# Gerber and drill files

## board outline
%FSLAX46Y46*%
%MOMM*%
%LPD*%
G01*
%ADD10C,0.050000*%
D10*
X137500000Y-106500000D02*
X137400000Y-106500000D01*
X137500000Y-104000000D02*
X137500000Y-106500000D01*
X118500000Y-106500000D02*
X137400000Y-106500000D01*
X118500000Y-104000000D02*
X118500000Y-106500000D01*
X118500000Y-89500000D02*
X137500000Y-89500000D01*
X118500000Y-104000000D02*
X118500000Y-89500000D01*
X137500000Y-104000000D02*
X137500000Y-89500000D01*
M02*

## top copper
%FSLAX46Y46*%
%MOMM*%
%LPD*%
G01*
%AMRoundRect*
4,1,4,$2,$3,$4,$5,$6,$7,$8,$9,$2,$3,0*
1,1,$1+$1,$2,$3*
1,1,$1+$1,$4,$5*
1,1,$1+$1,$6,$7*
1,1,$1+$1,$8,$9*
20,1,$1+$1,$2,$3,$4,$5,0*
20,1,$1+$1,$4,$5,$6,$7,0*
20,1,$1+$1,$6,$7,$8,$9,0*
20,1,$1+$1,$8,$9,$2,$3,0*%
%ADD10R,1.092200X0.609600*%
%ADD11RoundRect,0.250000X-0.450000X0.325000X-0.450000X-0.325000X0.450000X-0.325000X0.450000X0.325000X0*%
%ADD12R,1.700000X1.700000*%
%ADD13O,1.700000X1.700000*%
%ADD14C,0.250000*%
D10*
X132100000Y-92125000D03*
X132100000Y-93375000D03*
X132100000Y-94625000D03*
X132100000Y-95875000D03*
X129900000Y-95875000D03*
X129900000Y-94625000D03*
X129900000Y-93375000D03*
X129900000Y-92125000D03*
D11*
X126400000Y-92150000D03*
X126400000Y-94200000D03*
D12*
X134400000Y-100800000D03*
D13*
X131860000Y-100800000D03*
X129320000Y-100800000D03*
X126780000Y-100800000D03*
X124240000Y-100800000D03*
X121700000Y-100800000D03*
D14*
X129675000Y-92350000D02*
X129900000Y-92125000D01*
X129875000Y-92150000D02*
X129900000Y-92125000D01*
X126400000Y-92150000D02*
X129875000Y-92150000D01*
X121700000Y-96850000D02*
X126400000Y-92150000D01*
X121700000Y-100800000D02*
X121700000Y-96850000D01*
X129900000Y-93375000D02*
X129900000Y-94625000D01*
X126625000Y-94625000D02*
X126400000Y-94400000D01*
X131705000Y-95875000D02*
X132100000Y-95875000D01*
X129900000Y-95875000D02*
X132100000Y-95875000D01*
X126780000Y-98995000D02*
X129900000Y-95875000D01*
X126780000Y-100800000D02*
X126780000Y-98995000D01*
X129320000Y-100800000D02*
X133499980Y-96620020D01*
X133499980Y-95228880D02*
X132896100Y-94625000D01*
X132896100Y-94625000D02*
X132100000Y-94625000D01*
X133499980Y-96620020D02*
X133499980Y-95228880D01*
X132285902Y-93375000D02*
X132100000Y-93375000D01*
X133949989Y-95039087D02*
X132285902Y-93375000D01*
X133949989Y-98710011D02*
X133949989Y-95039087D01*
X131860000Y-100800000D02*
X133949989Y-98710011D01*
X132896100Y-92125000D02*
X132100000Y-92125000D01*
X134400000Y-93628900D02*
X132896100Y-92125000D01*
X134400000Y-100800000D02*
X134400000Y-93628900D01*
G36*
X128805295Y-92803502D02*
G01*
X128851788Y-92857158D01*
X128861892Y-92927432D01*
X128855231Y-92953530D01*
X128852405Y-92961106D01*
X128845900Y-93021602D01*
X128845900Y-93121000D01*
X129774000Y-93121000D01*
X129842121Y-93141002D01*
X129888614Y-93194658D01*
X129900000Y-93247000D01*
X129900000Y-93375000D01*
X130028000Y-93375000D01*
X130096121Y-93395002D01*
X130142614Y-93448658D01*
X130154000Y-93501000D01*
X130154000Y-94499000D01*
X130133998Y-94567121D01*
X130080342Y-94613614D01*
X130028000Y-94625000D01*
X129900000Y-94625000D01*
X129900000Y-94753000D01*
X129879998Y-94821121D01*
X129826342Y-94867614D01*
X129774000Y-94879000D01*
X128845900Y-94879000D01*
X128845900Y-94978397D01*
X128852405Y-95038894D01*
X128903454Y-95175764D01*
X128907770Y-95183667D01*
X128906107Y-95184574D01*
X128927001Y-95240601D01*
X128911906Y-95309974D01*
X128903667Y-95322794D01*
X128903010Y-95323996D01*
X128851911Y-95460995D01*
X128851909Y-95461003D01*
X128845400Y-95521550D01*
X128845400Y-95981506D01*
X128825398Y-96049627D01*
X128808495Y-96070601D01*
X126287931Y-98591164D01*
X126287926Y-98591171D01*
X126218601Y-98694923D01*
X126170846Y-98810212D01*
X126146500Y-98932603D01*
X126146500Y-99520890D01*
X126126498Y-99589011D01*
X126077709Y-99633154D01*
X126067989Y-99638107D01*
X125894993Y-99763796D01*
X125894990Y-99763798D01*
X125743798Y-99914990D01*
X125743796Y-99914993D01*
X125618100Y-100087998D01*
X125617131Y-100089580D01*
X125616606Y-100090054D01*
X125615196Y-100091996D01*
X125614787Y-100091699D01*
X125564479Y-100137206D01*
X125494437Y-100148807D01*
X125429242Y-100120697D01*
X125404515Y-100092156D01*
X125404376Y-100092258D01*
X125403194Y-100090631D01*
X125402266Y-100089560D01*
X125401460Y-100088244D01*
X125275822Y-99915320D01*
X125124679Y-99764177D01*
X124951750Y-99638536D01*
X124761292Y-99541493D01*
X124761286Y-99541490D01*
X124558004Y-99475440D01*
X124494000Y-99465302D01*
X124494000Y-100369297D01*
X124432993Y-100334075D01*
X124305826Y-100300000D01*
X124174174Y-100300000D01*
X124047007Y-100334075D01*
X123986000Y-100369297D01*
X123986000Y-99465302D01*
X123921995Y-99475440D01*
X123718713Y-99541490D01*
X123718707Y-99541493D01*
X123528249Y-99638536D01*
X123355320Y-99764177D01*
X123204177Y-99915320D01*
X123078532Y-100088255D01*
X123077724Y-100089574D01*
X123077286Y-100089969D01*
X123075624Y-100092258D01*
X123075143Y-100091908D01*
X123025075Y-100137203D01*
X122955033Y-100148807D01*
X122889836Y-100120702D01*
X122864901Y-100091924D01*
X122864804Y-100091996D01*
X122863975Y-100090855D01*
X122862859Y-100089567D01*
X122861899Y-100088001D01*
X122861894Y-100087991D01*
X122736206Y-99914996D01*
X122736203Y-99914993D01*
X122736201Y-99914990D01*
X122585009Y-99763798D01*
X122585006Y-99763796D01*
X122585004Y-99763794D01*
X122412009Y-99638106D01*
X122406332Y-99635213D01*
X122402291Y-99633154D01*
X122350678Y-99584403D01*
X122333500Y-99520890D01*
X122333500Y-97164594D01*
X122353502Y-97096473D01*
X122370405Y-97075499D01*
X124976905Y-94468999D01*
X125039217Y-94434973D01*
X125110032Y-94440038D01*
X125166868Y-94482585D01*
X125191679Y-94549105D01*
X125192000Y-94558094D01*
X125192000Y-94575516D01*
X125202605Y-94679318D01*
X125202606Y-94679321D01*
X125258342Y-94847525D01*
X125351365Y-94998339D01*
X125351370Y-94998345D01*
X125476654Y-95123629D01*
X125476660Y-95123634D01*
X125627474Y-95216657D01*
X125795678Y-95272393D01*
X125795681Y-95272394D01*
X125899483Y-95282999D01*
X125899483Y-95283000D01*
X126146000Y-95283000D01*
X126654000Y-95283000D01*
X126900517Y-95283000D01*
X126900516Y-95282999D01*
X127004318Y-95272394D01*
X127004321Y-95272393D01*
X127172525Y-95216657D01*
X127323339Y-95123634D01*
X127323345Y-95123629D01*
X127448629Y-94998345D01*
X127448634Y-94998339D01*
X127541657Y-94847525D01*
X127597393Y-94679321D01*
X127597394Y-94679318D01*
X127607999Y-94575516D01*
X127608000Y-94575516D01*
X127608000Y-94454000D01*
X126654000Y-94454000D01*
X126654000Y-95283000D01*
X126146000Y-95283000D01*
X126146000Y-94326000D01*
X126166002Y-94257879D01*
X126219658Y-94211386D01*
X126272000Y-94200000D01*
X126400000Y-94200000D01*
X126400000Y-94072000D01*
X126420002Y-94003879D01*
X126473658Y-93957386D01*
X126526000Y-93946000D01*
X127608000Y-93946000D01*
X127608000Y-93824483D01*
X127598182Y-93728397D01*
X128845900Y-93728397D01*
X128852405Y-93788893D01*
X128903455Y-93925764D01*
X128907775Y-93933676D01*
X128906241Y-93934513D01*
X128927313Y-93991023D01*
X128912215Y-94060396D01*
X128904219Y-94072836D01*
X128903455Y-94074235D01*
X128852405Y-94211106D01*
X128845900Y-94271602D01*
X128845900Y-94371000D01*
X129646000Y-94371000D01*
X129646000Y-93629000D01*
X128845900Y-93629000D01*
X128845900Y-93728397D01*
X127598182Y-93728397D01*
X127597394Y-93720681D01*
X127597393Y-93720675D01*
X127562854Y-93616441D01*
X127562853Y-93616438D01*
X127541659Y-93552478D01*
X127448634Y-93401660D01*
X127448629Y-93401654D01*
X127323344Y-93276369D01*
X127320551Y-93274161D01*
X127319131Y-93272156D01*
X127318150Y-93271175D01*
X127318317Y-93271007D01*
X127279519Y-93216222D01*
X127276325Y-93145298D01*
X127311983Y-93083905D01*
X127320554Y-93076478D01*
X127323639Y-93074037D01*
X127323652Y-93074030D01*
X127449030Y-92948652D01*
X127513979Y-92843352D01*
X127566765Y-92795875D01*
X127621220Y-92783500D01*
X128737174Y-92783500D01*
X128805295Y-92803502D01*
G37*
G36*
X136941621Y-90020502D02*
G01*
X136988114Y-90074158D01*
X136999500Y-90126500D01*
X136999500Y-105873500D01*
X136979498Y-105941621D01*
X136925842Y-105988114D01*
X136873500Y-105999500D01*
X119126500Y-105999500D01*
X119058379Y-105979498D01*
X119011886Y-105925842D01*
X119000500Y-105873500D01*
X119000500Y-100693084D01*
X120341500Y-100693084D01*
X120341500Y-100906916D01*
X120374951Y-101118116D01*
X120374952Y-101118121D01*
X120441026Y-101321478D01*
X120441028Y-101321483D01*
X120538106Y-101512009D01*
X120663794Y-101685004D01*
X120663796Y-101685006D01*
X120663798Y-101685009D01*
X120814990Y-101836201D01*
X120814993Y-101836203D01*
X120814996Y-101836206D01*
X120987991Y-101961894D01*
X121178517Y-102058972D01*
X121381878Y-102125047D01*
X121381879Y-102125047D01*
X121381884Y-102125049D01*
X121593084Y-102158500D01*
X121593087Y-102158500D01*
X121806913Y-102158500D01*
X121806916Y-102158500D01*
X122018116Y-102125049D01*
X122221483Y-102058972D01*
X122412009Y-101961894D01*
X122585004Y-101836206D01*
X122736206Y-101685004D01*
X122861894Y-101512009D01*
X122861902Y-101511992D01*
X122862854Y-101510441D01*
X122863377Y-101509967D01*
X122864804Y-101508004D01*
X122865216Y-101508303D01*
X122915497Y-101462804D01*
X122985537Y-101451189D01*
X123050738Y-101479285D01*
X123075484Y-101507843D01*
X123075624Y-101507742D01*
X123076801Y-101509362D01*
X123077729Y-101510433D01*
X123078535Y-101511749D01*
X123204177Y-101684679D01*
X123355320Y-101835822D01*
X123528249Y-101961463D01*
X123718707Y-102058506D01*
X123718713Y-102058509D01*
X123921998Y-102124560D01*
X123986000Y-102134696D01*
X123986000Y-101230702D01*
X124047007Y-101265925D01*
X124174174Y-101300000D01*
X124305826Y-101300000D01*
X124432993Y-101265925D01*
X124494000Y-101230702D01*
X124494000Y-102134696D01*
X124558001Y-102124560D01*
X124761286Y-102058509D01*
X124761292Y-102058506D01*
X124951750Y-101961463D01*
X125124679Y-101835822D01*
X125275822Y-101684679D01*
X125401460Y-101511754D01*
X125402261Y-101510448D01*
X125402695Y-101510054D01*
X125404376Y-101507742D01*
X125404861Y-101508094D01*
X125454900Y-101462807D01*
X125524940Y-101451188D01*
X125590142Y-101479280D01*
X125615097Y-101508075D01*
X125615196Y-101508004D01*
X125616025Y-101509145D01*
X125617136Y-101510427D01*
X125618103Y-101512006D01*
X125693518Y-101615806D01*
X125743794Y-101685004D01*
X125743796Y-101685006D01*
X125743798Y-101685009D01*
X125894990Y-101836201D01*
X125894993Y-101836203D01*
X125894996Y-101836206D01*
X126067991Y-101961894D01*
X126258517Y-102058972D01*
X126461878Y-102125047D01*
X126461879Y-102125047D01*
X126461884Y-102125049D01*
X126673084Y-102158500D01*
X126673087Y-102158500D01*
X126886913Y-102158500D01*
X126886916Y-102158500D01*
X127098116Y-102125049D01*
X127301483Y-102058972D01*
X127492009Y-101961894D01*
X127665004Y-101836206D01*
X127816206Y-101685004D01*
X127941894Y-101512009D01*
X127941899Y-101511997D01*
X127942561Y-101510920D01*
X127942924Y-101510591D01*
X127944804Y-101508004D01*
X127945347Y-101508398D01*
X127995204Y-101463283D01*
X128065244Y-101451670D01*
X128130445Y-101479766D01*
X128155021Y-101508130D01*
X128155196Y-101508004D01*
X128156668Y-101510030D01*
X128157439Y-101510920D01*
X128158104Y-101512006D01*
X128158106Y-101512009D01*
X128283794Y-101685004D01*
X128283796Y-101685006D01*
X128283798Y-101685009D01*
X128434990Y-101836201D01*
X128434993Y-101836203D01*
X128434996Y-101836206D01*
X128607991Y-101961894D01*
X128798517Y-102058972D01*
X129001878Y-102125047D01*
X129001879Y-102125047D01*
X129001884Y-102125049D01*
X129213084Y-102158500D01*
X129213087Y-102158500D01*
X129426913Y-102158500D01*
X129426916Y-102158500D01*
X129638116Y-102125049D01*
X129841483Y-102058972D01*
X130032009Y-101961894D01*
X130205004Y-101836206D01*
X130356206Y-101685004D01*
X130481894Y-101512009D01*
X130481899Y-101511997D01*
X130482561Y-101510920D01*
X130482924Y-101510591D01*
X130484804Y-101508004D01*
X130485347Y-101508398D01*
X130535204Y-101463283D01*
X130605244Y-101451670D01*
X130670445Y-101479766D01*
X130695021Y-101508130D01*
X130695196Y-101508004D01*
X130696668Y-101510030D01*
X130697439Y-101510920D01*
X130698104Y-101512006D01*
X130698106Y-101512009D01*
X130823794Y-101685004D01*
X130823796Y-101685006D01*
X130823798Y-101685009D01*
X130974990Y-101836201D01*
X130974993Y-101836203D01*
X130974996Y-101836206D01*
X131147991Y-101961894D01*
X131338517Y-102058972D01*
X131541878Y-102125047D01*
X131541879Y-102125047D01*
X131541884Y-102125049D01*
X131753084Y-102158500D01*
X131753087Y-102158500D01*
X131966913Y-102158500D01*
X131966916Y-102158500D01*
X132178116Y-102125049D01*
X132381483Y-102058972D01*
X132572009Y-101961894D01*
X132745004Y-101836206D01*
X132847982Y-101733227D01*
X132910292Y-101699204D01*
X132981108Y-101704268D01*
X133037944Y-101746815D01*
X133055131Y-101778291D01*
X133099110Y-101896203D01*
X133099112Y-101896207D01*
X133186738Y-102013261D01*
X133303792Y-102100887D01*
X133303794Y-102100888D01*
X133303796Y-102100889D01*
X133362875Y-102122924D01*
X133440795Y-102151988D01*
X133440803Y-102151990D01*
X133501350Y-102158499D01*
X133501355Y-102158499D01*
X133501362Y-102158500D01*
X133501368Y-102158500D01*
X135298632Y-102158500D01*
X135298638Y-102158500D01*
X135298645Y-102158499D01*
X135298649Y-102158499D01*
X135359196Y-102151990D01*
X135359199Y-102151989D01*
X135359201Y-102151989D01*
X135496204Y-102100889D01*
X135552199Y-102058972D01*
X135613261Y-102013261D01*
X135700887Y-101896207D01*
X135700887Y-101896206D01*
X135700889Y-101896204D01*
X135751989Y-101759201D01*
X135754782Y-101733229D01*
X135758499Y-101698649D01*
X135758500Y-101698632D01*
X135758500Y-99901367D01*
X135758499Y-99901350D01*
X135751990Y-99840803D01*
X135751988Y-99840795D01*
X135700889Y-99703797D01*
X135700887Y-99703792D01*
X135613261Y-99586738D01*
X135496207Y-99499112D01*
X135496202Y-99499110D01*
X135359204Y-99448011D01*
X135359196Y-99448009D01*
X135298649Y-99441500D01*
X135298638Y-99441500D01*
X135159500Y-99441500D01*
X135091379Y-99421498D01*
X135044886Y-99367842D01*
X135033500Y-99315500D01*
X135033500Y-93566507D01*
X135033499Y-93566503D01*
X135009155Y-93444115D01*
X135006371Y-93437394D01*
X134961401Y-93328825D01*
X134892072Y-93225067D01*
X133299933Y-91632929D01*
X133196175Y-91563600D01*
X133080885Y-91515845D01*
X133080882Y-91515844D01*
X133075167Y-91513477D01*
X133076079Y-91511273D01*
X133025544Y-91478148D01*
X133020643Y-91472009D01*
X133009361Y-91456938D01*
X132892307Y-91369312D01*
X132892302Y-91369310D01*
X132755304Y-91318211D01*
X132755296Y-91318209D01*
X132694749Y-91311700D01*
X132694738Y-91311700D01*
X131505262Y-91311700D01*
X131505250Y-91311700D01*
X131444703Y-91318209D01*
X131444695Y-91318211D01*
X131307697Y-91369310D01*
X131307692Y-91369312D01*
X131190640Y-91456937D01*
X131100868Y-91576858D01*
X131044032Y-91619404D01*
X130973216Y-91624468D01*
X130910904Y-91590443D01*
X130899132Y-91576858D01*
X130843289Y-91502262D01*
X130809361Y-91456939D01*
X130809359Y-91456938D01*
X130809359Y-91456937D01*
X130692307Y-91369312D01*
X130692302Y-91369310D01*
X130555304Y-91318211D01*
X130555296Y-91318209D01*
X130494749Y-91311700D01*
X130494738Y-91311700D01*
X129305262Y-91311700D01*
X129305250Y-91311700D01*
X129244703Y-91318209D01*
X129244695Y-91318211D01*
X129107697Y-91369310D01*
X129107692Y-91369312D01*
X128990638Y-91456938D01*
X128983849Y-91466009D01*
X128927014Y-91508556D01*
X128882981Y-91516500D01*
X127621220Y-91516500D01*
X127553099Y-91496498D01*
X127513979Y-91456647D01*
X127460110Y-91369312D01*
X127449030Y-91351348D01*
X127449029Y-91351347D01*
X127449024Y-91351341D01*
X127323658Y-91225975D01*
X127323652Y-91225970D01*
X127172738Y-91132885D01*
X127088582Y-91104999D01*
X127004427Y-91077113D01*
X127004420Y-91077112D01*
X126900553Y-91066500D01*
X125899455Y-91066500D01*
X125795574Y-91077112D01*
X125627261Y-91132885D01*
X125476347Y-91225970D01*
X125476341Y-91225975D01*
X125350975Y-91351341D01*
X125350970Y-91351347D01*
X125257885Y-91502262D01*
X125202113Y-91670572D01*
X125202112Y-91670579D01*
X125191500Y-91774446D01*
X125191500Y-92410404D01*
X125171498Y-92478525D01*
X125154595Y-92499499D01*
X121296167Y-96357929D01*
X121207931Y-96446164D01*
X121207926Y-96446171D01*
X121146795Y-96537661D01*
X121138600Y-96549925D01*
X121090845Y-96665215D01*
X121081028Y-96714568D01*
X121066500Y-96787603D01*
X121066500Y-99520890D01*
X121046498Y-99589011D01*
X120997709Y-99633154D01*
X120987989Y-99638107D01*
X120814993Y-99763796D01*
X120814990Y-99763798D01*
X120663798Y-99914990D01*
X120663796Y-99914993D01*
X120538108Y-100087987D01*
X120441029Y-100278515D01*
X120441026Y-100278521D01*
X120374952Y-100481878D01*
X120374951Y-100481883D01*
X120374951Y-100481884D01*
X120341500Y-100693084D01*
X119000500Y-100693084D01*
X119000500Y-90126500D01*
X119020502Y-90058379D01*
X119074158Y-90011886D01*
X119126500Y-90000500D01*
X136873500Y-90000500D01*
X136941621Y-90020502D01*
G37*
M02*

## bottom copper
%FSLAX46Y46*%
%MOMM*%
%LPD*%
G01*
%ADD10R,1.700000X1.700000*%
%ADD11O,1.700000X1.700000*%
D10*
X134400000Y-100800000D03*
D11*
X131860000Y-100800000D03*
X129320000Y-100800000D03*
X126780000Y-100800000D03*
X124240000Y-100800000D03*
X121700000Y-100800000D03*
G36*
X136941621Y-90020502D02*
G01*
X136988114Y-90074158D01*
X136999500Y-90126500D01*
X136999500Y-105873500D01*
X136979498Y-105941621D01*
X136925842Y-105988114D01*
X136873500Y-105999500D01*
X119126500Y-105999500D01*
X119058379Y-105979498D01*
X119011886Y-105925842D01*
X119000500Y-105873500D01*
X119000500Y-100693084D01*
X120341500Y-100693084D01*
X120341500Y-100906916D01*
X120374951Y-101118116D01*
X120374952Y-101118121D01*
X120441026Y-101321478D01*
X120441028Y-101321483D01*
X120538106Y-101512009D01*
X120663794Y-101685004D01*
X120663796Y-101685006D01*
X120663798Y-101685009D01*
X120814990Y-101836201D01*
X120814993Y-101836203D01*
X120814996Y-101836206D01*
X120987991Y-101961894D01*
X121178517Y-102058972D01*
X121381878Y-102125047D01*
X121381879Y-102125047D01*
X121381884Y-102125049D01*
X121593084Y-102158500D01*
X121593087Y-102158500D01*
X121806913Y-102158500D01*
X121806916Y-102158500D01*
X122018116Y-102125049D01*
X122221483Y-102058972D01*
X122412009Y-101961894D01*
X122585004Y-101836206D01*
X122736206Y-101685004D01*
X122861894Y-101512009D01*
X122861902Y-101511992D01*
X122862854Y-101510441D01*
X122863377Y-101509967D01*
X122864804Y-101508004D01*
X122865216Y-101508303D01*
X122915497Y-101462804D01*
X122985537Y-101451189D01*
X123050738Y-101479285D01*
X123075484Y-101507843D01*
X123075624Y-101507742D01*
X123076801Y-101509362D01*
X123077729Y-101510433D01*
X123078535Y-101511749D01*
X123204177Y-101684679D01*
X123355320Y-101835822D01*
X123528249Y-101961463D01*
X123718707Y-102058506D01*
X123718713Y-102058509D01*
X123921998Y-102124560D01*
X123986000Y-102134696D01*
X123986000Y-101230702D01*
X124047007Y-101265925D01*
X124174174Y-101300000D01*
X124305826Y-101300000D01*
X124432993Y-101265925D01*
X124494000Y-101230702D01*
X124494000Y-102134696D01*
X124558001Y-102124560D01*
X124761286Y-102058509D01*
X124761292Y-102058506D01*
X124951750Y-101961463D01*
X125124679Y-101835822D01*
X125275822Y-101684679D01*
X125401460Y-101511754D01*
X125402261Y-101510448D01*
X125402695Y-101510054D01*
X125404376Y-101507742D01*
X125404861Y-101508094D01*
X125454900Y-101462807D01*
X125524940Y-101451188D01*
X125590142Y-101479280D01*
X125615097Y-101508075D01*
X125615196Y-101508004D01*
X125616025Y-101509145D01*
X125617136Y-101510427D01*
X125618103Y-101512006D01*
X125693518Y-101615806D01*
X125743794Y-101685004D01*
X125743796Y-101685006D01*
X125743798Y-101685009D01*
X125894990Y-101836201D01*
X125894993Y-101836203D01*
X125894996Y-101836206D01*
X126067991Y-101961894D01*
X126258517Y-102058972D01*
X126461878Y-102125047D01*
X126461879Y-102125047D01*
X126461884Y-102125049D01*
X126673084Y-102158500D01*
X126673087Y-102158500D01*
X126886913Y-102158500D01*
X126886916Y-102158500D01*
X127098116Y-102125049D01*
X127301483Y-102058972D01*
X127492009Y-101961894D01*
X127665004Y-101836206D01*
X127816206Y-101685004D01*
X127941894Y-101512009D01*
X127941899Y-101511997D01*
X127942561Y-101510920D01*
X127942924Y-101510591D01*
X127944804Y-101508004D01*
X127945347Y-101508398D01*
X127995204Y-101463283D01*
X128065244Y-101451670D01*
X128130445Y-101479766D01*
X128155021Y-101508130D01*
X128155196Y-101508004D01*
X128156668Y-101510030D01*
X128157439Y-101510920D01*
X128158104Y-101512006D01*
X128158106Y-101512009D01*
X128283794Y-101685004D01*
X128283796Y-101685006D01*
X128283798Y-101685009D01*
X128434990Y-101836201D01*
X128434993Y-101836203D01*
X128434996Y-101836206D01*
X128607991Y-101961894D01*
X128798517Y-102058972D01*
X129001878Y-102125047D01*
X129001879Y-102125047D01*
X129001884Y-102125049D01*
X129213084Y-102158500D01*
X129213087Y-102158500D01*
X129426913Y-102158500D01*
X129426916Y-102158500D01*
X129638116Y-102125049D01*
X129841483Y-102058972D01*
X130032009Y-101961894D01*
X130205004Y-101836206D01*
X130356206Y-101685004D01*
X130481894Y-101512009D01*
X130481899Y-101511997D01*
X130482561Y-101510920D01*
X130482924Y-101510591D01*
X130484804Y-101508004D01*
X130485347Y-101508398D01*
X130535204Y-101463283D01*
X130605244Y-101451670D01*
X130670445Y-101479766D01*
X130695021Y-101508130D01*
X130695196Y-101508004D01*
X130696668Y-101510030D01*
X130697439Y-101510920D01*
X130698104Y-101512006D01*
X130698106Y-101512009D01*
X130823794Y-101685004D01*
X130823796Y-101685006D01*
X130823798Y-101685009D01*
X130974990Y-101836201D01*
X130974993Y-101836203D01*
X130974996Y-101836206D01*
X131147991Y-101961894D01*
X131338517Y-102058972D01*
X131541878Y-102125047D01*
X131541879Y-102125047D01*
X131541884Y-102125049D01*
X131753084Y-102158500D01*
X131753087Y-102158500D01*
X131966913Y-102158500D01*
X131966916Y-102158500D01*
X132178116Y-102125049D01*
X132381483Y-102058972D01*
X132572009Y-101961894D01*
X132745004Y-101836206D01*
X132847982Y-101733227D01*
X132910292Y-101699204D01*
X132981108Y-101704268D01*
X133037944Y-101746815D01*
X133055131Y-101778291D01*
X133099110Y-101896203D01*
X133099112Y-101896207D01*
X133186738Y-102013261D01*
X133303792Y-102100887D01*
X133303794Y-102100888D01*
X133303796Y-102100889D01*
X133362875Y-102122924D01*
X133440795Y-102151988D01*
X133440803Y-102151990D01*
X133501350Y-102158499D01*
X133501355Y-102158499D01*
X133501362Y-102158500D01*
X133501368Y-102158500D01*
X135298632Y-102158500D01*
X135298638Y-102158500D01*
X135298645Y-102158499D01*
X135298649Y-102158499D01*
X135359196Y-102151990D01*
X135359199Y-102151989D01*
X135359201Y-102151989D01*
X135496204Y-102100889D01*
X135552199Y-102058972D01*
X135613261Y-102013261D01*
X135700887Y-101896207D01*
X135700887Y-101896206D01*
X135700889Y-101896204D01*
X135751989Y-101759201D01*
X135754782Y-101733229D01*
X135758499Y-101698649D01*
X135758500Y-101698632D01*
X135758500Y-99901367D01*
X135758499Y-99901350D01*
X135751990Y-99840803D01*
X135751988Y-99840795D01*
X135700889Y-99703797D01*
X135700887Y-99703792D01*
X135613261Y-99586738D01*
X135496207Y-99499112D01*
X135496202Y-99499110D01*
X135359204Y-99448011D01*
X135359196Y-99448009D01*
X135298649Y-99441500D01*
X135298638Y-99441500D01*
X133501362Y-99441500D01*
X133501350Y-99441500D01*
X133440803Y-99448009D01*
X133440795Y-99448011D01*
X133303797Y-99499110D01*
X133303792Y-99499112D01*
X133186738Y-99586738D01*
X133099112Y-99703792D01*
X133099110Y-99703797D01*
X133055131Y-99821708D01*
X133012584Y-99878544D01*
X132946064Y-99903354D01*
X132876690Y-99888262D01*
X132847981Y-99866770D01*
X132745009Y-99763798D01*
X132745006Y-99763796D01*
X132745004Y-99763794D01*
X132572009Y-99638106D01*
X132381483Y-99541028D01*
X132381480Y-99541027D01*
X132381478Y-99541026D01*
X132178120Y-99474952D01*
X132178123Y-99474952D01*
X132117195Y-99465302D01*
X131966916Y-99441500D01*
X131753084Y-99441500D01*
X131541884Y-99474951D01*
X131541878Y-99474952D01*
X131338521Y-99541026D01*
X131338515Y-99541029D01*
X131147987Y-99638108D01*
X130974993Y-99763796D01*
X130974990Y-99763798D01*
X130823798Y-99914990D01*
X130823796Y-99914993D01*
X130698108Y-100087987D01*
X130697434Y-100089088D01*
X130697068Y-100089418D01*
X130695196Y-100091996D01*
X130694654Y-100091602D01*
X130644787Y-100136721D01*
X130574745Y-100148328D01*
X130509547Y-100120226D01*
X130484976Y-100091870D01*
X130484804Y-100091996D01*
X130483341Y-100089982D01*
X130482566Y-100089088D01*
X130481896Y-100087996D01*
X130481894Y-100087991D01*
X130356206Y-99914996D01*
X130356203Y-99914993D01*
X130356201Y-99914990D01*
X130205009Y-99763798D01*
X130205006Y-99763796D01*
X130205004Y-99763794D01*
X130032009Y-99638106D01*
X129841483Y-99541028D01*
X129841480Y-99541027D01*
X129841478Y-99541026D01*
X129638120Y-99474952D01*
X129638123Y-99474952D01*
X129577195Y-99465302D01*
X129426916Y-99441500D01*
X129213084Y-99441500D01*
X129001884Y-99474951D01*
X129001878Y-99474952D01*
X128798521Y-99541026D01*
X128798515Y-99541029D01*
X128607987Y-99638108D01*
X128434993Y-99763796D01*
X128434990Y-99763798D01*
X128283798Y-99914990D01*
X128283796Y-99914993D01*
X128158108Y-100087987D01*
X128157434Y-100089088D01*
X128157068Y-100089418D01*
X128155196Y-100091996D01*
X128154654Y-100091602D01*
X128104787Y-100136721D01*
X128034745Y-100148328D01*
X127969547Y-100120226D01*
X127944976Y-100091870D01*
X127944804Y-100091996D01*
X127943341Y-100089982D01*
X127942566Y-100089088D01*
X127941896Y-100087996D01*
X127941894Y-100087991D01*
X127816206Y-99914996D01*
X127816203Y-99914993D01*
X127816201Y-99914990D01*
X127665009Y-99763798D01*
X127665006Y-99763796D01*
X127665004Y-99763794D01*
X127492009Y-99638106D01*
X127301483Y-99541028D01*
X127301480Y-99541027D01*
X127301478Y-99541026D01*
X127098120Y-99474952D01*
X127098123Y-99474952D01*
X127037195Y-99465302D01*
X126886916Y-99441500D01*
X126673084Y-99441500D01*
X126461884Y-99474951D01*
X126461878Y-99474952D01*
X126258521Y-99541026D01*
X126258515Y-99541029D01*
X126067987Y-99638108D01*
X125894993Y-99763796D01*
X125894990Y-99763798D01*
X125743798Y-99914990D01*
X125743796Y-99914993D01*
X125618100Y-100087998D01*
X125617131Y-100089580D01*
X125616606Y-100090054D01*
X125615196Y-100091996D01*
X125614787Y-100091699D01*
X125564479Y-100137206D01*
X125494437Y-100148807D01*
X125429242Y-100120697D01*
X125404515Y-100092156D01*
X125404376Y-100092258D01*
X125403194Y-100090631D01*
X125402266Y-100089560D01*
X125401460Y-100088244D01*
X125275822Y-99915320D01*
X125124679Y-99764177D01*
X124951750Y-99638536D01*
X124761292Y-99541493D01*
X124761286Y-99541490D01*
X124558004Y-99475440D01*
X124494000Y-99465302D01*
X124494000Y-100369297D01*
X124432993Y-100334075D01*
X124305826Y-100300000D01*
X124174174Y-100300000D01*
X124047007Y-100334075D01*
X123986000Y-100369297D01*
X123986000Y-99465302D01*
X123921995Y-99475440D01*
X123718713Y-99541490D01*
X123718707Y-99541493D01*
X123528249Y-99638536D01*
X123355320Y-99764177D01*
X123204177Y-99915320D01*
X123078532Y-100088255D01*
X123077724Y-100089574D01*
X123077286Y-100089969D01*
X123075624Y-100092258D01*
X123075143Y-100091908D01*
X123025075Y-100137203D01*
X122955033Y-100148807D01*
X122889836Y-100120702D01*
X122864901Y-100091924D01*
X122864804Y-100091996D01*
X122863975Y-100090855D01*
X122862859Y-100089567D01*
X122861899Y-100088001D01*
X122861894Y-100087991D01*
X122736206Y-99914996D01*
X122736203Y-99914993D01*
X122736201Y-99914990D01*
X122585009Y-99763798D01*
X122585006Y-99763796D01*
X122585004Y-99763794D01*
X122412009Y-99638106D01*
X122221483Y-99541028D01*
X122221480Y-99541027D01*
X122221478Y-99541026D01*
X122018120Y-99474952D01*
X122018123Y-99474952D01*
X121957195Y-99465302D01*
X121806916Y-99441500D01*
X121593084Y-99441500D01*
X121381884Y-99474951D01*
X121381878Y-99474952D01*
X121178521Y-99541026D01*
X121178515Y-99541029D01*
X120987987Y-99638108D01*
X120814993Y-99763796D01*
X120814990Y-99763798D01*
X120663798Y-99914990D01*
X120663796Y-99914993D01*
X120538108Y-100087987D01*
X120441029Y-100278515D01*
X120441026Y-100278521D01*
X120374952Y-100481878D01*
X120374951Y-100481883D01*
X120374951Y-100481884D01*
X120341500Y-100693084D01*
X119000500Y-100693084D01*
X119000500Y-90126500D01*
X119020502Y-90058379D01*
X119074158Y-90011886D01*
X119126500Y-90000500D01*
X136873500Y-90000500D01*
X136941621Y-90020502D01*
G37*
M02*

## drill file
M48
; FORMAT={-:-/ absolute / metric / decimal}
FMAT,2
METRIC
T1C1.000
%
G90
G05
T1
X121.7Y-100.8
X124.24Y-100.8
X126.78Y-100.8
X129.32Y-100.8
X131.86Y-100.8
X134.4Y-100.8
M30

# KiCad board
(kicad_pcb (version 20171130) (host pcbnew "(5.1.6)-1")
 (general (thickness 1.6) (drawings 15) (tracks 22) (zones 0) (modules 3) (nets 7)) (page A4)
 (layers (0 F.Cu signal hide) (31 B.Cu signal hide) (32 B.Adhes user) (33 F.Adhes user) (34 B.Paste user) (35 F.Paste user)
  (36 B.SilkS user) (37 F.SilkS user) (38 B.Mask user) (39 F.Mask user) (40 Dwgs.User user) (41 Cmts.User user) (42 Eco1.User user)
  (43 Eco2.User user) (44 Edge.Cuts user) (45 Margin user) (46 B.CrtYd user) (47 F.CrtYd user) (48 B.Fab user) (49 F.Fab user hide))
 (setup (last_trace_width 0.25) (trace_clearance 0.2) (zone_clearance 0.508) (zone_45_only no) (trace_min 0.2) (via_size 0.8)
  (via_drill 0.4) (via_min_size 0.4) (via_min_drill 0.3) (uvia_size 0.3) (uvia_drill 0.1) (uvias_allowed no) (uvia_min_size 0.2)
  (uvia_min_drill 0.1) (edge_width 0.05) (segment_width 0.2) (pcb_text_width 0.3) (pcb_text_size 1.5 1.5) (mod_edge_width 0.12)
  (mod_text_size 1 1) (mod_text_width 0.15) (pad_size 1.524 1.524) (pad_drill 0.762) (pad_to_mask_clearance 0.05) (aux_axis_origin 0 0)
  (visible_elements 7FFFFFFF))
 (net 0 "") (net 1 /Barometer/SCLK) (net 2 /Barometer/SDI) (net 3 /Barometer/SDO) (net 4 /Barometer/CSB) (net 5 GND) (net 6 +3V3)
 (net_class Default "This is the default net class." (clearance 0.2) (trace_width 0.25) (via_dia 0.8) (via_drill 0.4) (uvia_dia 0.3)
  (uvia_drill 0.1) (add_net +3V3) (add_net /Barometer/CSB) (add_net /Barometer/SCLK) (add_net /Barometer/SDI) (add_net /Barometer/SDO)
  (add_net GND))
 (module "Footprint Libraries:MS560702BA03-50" (layer F.Cu) (at 131 94)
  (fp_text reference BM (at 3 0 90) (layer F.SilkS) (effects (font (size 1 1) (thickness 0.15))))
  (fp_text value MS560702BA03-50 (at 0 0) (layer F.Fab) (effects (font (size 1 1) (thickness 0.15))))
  (pad 8 smd rect (at 1.1 -1.875) (size 1.0922 0.6096) (layers F.Cu F.Paste F.Mask) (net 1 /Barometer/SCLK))
  (pad 7 smd rect (at 1.1 -0.625) (size 1.0922 0.6096) (layers F.Cu F.Paste F.Mask) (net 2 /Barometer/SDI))
  (pad 6 smd rect (at 1.1 0.625) (size 1.0922 0.6096) (layers F.Cu F.Paste F.Mask) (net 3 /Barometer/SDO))
  (pad 5 smd rect (at 1.1 1.875) (size 1.0922 0.6096) (layers F.Cu F.Paste F.Mask) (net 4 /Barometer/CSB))
  (pad 4 smd rect (at -1.1 1.875) (size 1.0922 0.6096) (layers F.Cu F.Paste F.Mask) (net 4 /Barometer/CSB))
  (pad 3 smd rect (at -1.1 0.625) (size 1.0922 0.6096) (layers F.Cu F.Paste F.Mask) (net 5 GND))
  (pad 2 smd rect (at -1.1 -0.625) (size 1.0922 0.6096) (layers F.Cu F.Paste F.Mask) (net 5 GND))
  (pad 1 smd rect (at -1.1 -1.875) (size 1.0922 0.6096) (layers F.Cu F.Paste F.Mask) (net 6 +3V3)))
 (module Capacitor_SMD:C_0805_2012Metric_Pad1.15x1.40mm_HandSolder (layer F.Cu) (at 126.4 93.175 270)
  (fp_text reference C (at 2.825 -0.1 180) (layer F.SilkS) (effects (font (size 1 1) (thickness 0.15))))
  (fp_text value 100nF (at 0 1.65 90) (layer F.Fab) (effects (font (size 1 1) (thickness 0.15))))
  (pad 1 smd roundrect (at -1.025 0 270) (size 1.15 1.4) (layers F.Cu F.Paste F.Mask) (roundrect_rratio 0.217391) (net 6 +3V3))
  (pad 2 smd roundrect (at 1.025 0 270) (size 1.15 1.4) (layers F.Cu F.Paste F.Mask) (roundrect_rratio 0.217391) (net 5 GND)))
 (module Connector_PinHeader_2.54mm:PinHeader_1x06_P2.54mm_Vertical (layer F.Cu) (at 134.4 100.8 270)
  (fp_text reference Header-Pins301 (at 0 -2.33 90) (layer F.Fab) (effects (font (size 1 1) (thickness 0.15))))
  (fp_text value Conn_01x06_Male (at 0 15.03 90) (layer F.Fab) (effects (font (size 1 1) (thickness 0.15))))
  (pad 1 thru_hole rect (at 0 0 270) (size 1.7 1.7) (drill 1) (layers *.Cu *.Mask) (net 1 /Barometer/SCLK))
  (pad 2 thru_hole oval (at 0 2.54 270) (size 1.7 1.7) (drill 1) (layers *.Cu *.Mask) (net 2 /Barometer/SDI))
  (pad 3 thru_hole oval (at 0 5.08 270) (size 1.7 1.7) (drill 1) (layers *.Cu *.Mask) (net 3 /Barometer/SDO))
  (pad 4 thru_hole oval (at 0 7.62 270) (size 1.7 1.7) (drill 1) (layers *.Cu *.Mask) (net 4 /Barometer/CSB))
  (pad 5 thru_hole oval (at 0 10.16 270) (size 1.7 1.7) (drill 1) (layers *.Cu *.Mask) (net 5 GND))
  (pad 6 thru_hole oval (at 0 12.7 270) (size 1.7 1.7) (drill 1) (layers *.Cu *.Mask) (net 6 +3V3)))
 (gr_line (start 137.5 106.5) (end 137.4 106.5) (layer Edge.Cuts) (width 0.05))
 (gr_line (start 137.5 104) (end 137.5 106.5) (layer Edge.Cuts) (width 0.05))
 (gr_line (start 118.5 106.5) (end 137.4 106.5) (layer Edge.Cuts) (width 0.05))
 (gr_line (start 118.5 104) (end 118.5 106.5) (layer Edge.Cuts) (width 0.05))
 (gr_line (start 118.5 89.5) (end 137.5 89.5) (layer Edge.Cuts) (width 0.05))
 (gr_line (start 118.5 104) (end 118.5 89.5) (layer Edge.Cuts) (width 0.05))
 (gr_line (start 137.5 104) (end 137.5 89.5) (layer Edge.Cuts) (width 0.05))
 (segment (start 129.675 92.35) (end 129.9 92.125) (width 0.25) (layer F.Cu) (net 6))
 (segment (start 129.875 92.15) (end 129.9 92.125) (width 0.25) (layer F.Cu) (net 6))
 (segment (start 126.4 92.15) (end 129.875 92.15) (width 0.25) (layer F.Cu) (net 6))
 (segment (start 121.7 96.85) (end 126.4 92.15) (width 0.25) (layer F.Cu) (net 6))
 (segment (start 121.7 100.8) (end 121.7 96.85) (width 0.25) (layer F.Cu) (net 6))
 (segment (start 129.9 93.375) (end 129.9 94.625) (width 0.25) (layer F.Cu) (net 5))
 (segment (start 126.625 94.625) (end 126.4 94.4) (width 0.25) (layer F.Cu) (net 5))
 (segment (start 131.705 95.875) (end 132.1 95.875) (width 0.25) (layer F.Cu) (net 4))
 (segment (start 129.9 95.875) (end 132.1 95.875) (width 0.25) (layer F.Cu) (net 4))
 (segment (start 126.78 98.995) (end 129.9 95.875) (width 0.25) (layer F.Cu) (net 4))
 (segment (start 126.78 100.8) (end 126.78 98.995) (width 0.25) (layer F.Cu) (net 4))
 (segment (start 129.32 100.8) (end 133.49998 96.62002) (width 0.25) (layer F.Cu) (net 3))
 (segment (start 133.49998 95.22888) (end 132.8961 94.625) (width 0.25) (layer F.Cu) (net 3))
 (segment (start 132.8961 94.625) (end 132.1 94.625) (width 0.25) (layer F.Cu) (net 3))
 (segment (start 133.49998 96.62002) (end 133.49998 95.22888) (width 0.25) (layer F.Cu) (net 3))
 (segment (start 132.285902 93.375) (end 132.1 93.375) (width 0.25) (layer F.Cu) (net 2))
 (segment (start 133.949989 95.039087) (end 132.285902 93.375) (width 0.25) (layer F.Cu) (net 2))
 (segment (start 133.949989 98.710011) (end 133.949989 95.039087) (width 0.25) (layer F.Cu) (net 2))
 (segment (start 131.86 100.8) (end 133.949989 98.710011) (width 0.25) (layer F.Cu) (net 2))
 (segment (start 132.8961 92.125) (end 132.1 92.125) (width 0.25) (layer F.Cu) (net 1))
 (segment (start 134.4 93.6289) (end 132.8961 92.125) (width 0.25) (layer F.Cu) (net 1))
 (segment (start 134.4 100.8) (end 134.4 93.6289) (width 0.25) (layer F.Cu) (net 1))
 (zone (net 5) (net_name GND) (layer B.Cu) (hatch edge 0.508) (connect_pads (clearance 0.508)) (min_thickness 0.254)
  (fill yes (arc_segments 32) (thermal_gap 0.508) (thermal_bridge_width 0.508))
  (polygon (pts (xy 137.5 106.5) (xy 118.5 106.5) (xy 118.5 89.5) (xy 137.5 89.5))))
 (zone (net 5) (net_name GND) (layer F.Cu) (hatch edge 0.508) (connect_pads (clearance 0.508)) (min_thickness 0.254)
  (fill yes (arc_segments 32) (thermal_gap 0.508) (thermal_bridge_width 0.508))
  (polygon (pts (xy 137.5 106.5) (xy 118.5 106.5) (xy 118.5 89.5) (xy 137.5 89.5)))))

